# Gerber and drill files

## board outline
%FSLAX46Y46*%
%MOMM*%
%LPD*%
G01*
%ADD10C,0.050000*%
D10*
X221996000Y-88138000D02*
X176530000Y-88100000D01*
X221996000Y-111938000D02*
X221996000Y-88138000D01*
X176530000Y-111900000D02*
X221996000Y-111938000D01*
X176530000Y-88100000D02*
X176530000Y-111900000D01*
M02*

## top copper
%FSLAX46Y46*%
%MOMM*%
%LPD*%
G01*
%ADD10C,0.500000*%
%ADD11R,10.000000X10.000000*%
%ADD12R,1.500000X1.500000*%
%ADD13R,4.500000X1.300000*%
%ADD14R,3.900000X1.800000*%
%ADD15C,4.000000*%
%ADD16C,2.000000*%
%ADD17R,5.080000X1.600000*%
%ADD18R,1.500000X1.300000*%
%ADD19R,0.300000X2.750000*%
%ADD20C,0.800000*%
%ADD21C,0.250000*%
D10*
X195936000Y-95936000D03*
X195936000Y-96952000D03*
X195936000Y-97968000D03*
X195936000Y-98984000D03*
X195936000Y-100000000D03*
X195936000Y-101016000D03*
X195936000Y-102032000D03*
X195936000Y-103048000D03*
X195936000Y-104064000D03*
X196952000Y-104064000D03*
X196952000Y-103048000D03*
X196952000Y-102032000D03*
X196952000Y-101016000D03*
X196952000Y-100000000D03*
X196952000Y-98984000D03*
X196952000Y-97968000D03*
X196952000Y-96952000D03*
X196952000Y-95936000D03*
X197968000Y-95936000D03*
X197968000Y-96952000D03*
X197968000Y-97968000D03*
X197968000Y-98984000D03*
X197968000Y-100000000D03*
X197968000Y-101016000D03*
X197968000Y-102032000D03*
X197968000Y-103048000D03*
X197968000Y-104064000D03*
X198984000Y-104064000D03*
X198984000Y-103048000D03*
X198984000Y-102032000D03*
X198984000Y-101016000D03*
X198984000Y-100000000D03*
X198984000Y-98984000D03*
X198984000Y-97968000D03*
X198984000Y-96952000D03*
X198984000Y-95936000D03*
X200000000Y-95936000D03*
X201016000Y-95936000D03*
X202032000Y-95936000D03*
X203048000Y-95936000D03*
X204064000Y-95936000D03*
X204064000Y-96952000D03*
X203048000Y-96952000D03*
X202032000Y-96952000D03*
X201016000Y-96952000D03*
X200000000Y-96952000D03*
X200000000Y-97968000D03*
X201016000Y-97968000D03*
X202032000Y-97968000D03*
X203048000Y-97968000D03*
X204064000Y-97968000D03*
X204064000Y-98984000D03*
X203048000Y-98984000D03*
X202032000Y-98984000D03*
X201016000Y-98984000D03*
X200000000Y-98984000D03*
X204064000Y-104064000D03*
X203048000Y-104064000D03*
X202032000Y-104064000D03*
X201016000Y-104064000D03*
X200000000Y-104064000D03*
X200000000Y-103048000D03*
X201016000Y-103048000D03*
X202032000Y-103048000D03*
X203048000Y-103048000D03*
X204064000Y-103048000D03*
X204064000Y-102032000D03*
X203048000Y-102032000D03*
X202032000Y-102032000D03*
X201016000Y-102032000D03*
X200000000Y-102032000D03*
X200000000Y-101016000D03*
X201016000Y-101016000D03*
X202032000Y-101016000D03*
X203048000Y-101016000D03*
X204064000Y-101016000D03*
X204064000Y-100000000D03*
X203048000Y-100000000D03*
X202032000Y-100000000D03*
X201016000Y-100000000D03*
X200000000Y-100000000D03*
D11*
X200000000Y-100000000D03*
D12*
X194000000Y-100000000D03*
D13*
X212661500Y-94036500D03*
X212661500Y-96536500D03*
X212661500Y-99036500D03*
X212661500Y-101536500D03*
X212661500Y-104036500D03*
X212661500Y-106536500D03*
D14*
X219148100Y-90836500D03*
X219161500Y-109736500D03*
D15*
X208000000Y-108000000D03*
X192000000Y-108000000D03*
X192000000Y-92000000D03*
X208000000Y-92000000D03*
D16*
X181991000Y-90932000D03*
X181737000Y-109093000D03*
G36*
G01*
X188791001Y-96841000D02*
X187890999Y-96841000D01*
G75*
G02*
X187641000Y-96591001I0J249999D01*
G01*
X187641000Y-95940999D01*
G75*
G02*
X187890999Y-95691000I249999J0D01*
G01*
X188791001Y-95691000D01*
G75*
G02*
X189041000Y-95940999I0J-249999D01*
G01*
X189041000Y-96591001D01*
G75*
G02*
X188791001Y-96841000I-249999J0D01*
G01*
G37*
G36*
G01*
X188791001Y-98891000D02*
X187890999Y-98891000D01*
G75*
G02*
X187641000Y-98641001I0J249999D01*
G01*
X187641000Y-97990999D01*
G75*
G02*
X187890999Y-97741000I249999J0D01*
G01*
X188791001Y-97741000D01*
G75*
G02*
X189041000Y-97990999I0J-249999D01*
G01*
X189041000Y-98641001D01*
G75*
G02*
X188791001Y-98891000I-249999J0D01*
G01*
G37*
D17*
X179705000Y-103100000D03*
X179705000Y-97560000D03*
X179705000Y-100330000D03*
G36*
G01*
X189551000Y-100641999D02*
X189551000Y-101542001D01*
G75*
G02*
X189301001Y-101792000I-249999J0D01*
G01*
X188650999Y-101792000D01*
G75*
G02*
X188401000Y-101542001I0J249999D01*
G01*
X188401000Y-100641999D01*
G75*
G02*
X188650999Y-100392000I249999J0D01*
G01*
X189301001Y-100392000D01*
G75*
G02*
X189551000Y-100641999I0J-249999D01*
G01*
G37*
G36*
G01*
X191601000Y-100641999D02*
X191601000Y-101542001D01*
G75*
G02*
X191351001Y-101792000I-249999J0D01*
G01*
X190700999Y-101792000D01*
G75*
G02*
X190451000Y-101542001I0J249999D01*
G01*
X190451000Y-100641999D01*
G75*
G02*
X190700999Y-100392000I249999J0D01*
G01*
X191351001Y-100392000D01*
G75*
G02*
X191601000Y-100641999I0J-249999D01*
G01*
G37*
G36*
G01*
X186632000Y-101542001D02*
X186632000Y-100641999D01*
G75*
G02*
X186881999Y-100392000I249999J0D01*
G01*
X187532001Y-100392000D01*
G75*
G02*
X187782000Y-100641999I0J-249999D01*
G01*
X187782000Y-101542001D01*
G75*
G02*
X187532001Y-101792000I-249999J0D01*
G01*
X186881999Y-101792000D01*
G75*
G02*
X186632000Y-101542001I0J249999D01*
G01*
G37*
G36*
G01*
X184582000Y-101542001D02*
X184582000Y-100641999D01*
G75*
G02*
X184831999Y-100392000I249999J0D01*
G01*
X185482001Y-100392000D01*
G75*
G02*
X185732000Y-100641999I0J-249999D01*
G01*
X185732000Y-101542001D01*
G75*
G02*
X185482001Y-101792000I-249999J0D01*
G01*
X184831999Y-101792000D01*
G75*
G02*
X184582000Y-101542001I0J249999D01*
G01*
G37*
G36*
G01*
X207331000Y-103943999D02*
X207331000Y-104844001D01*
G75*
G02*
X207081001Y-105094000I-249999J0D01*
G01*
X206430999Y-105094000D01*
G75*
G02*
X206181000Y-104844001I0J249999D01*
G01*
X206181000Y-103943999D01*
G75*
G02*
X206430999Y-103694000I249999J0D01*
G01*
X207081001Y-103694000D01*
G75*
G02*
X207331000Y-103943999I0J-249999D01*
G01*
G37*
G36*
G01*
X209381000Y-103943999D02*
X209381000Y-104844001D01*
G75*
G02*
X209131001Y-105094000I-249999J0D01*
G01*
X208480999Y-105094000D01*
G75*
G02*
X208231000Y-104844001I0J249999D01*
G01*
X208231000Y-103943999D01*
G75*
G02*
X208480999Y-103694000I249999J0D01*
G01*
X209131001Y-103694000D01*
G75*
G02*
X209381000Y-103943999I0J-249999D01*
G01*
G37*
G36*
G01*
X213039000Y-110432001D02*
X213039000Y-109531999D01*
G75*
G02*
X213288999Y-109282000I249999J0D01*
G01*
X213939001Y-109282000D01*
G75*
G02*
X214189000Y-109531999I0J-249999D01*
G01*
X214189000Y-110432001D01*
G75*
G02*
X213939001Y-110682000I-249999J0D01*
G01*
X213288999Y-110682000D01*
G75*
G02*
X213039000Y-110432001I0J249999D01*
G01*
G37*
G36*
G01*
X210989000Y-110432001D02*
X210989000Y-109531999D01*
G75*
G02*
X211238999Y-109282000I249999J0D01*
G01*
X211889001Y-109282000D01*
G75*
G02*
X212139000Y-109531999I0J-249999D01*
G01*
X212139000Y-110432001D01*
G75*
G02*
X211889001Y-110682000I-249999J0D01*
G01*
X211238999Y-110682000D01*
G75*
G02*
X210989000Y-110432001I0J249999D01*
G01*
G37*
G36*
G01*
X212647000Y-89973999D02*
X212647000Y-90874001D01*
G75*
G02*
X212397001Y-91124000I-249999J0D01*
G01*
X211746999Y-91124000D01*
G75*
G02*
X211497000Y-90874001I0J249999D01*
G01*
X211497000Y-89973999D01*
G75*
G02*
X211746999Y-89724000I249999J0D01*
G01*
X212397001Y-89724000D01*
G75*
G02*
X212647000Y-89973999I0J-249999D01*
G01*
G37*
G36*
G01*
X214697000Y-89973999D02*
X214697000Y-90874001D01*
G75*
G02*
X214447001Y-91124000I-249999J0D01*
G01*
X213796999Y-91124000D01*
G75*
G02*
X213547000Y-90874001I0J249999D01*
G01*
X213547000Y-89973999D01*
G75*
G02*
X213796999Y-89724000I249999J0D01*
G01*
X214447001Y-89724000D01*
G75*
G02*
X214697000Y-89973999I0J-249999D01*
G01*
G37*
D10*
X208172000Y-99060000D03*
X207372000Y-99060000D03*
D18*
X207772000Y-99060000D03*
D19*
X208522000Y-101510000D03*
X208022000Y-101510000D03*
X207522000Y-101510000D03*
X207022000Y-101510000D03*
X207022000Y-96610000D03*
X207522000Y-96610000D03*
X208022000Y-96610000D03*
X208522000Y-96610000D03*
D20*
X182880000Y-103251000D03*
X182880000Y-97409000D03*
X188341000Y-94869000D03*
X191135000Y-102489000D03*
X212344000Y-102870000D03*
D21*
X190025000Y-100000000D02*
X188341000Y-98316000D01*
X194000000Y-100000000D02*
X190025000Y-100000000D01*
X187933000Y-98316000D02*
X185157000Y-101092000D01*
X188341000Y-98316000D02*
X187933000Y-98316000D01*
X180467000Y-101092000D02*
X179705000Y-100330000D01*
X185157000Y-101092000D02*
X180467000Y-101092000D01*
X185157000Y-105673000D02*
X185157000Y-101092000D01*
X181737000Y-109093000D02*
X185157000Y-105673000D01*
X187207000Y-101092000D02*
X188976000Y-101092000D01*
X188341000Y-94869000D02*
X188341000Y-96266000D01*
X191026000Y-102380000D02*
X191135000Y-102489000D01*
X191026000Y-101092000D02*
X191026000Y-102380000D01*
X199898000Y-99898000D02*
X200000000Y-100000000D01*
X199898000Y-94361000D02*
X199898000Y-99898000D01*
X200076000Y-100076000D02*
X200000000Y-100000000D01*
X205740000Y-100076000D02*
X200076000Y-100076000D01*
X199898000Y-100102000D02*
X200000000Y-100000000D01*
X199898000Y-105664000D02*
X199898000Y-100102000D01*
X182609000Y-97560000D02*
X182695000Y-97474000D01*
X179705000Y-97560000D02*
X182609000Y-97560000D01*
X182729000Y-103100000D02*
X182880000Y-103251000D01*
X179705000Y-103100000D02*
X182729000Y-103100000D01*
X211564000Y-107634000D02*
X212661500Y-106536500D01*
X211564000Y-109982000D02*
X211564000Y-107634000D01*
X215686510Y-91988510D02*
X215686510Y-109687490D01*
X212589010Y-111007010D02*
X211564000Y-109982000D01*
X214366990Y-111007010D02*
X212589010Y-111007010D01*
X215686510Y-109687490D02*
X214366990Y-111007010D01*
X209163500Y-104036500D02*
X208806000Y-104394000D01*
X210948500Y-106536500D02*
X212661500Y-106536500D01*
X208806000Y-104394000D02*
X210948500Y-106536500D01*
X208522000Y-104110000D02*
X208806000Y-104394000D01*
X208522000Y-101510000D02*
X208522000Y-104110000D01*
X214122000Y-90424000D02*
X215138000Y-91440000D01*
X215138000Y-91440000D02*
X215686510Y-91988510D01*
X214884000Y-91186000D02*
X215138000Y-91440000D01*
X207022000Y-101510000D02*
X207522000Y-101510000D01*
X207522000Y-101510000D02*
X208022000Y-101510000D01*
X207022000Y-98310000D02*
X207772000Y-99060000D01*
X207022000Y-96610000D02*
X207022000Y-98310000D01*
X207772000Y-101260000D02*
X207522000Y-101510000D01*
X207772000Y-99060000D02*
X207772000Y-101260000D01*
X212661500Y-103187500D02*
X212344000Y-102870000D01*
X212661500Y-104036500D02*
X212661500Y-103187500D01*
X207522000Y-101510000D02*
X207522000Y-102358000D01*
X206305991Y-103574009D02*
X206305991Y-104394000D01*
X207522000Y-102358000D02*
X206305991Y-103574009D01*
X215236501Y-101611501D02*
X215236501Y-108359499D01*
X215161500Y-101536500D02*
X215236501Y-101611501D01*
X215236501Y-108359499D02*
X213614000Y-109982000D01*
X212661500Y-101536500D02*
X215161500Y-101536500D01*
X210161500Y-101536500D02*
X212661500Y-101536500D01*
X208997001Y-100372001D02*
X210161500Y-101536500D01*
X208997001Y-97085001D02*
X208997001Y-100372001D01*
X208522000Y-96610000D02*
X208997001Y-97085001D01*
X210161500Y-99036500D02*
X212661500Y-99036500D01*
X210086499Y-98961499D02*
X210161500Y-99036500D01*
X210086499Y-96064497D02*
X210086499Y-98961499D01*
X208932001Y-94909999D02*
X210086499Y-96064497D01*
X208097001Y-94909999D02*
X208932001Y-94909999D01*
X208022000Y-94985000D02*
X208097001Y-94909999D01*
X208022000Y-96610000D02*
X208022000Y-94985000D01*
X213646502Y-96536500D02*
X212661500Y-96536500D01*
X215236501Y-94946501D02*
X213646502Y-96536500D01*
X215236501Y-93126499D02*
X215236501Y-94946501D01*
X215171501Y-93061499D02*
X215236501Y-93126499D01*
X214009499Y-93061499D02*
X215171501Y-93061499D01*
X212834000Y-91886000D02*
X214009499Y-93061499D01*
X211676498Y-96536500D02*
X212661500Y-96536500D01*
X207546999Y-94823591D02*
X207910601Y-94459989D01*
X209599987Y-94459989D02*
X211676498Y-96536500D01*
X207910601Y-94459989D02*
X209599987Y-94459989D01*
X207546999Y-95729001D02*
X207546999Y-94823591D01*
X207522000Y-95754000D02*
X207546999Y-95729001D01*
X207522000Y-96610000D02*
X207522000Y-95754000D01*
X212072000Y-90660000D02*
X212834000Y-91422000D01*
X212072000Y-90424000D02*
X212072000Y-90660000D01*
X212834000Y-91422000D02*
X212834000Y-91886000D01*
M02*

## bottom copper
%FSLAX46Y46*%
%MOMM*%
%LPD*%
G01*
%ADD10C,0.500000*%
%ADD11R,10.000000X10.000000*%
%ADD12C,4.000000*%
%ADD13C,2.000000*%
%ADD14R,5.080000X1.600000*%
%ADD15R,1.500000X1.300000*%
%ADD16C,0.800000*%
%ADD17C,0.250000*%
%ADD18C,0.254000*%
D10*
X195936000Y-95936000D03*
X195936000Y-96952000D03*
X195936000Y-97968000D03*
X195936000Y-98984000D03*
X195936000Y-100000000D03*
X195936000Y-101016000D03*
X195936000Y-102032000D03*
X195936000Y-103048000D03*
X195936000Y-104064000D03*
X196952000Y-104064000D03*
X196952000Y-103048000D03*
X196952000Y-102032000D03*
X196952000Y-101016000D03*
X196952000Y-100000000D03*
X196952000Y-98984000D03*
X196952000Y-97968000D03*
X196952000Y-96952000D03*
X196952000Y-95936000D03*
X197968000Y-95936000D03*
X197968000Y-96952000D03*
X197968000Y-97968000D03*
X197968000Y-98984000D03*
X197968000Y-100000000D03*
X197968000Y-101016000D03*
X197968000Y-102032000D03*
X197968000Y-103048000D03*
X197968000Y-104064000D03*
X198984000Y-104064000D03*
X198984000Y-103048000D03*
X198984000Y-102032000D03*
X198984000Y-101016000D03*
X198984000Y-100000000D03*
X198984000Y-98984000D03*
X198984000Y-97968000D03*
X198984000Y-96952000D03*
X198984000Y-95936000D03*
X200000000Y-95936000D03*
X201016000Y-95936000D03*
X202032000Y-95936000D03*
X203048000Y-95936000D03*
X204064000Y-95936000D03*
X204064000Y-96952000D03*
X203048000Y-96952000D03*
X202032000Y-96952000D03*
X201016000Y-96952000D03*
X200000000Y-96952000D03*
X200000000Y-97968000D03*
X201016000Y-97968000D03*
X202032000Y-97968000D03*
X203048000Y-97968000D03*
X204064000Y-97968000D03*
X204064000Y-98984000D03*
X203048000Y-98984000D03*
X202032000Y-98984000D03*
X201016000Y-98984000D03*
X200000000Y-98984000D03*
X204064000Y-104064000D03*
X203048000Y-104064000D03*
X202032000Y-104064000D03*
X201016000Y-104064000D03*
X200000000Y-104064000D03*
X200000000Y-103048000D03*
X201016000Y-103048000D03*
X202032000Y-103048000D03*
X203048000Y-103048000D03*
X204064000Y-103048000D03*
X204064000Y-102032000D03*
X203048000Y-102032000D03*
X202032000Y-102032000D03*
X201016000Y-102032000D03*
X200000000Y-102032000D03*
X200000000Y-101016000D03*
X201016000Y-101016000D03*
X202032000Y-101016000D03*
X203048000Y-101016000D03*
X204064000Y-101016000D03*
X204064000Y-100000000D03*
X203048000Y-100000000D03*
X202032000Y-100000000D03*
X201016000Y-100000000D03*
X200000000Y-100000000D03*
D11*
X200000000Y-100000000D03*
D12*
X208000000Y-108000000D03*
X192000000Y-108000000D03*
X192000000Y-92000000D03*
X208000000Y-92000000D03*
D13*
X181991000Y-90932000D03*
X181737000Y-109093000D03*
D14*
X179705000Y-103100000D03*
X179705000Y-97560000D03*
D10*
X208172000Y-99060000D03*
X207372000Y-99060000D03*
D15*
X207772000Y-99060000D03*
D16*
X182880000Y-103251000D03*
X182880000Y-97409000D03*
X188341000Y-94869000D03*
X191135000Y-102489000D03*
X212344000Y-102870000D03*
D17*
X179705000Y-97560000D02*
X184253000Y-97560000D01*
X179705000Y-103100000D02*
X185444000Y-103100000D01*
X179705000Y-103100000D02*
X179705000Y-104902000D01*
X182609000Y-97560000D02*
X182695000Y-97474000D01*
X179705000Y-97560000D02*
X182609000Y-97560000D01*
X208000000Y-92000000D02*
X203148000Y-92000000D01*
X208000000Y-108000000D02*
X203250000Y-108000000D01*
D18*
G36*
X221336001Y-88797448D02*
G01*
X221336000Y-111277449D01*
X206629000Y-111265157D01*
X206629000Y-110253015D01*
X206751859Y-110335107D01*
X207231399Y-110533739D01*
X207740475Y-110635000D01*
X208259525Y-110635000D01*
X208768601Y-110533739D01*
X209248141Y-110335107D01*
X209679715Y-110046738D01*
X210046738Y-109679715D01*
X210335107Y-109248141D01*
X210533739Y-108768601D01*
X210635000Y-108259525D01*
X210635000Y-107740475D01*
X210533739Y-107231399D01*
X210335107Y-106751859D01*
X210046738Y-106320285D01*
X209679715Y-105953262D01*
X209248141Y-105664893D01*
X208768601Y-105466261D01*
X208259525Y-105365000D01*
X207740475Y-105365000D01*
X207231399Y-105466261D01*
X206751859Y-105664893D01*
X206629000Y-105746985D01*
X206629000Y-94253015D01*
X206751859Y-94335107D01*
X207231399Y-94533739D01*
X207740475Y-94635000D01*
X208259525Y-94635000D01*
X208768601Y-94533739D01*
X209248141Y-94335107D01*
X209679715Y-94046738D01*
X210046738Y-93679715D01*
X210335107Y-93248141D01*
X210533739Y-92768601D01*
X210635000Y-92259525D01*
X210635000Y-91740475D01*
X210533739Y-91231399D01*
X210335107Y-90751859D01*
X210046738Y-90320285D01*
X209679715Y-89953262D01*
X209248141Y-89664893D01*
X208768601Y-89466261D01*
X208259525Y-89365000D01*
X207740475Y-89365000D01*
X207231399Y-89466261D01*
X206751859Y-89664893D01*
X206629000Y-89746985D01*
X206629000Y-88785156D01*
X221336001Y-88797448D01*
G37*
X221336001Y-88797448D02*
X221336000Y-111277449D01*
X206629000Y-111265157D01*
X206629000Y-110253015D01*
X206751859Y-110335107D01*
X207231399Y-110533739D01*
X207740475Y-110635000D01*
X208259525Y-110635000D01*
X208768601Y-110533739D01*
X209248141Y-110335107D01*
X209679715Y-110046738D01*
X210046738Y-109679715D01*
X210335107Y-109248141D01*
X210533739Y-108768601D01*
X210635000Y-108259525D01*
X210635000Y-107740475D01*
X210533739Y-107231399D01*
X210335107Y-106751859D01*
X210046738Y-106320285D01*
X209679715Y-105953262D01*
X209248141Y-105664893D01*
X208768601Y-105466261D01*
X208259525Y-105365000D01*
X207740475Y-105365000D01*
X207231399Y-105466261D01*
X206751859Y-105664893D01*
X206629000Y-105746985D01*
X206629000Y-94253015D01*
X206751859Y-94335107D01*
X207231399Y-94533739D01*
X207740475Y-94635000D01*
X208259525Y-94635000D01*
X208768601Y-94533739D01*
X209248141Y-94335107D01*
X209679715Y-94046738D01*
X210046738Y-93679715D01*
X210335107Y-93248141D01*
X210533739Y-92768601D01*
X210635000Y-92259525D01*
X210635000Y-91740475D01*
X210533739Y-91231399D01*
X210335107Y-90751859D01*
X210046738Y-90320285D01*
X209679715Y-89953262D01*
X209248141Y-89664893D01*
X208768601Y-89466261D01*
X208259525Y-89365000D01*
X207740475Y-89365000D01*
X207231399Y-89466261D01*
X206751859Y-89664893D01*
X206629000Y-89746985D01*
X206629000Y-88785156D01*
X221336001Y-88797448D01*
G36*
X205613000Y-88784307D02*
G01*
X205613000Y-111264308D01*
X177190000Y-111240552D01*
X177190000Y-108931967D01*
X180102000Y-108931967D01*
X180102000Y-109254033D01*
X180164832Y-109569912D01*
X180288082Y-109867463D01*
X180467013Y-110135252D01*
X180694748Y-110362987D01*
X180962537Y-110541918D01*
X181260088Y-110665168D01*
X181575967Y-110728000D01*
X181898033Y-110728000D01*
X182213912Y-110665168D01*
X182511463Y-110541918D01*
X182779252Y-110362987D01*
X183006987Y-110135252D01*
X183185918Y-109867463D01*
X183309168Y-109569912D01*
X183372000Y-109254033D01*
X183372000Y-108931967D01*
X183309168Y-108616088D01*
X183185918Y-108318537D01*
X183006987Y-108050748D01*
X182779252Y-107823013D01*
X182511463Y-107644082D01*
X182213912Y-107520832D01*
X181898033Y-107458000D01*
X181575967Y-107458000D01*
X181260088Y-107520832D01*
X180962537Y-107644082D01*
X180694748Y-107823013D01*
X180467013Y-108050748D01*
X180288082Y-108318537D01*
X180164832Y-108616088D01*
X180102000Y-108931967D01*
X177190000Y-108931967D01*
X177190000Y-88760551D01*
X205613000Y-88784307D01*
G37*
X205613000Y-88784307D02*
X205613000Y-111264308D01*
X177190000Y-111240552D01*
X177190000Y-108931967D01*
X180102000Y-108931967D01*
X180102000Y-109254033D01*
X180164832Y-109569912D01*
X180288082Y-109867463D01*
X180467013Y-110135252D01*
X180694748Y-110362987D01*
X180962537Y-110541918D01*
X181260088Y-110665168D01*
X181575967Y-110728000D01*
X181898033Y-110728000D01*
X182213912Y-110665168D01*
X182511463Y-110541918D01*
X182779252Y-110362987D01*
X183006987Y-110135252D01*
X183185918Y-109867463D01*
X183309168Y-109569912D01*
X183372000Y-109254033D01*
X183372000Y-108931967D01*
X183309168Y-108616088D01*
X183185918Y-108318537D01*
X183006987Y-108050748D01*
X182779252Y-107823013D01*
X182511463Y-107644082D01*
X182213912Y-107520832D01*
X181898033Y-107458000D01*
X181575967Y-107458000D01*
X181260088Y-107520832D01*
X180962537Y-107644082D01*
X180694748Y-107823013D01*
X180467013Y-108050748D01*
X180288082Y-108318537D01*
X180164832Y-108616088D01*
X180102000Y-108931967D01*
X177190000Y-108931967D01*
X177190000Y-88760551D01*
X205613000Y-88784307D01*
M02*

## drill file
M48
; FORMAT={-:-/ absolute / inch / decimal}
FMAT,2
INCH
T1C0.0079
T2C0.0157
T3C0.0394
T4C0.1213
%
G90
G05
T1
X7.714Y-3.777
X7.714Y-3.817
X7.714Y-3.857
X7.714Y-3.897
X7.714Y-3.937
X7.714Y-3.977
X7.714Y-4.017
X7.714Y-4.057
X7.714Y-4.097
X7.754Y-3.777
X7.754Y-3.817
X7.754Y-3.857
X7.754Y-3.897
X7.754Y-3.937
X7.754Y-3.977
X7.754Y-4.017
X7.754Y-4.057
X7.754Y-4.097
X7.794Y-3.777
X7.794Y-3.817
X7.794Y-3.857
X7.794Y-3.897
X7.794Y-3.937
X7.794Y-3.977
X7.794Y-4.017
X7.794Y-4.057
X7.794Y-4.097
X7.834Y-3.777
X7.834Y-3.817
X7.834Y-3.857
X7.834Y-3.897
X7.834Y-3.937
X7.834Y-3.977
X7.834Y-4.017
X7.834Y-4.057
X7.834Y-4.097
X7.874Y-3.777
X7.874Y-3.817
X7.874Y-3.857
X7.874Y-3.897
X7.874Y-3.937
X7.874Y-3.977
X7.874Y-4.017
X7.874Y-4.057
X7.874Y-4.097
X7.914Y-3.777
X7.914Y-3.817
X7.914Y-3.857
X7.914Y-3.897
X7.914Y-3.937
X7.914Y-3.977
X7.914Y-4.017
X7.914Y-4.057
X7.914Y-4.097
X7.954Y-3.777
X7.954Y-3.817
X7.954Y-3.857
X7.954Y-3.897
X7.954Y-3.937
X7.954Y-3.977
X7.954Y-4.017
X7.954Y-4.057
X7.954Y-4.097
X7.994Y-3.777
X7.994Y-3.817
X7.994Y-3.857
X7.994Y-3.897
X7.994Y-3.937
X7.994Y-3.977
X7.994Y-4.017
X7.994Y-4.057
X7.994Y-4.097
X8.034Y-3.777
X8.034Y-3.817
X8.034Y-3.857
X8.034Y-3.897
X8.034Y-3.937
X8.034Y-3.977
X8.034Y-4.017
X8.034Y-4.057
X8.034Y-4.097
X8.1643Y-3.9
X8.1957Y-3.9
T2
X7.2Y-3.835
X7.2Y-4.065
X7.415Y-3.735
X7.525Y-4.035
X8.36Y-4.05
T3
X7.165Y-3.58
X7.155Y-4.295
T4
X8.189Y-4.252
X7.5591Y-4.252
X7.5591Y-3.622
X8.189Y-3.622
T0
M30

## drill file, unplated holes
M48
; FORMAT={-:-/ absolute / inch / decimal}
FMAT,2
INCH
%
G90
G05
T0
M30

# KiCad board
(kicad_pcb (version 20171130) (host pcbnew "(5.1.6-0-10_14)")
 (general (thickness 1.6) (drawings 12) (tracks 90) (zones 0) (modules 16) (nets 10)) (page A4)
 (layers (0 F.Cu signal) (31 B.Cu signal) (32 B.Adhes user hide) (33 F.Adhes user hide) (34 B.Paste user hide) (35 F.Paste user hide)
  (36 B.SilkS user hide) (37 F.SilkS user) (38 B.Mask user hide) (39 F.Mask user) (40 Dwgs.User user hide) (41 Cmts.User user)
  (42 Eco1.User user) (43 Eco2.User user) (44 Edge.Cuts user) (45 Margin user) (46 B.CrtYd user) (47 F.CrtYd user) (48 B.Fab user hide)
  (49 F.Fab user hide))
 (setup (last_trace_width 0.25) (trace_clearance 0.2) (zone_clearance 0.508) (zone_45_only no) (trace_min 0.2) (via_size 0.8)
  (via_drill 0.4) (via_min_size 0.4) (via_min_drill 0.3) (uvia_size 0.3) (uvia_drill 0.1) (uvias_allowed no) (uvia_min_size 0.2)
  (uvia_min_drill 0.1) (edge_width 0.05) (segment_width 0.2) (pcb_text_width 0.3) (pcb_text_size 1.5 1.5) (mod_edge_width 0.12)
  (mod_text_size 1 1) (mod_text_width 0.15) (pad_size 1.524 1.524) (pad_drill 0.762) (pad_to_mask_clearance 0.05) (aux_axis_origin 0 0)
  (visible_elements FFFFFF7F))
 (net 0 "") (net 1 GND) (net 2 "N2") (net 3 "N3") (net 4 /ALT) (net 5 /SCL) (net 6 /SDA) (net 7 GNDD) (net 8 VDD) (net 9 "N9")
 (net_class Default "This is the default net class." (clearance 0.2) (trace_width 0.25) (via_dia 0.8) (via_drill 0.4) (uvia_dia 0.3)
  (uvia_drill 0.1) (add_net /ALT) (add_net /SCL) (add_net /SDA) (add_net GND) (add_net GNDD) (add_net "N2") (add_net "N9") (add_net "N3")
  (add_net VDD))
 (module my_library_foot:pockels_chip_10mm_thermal (layer F.Cu) (at 200 100)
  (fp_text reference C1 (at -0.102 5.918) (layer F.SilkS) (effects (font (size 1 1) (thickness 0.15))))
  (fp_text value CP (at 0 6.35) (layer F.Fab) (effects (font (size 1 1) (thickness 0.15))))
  (pad 2 thru_hole circle (at -4.064 -4.064) (size 0.5 0.5) (drill 0.2) (layers *.Cu *.Mask) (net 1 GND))
  (pad 2 thru_hole circle (at -4.064 -3.048) (size 0.5 0.5) (drill 0.2) (layers *.Cu *.Mask) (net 1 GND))
  (pad 2 thru_hole circle (at -4.064 -2.032) (size 0.5 0.5) (drill 0.2) (layers *.Cu *.Mask) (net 1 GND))
  (pad 2 thru_hole circle (at -4.064 -1.016) (size 0.5 0.5) (drill 0.2) (layers *.Cu *.Mask) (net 1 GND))
  (pad 2 thru_hole circle (at -4.064 0) (size 0.5 0.5) (drill 0.2) (layers *.Cu *.Mask) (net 1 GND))
  (pad 2 thru_hole circle (at -4.064 1.016) (size 0.5 0.5) (drill 0.2) (layers *.Cu *.Mask) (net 1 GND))
  (pad 2 thru_hole circle (at -4.064 2.032) (size 0.5 0.5) (drill 0.2) (layers *.Cu *.Mask) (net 1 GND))
  (pad 2 thru_hole circle (at -4.064 3.048) (size 0.5 0.5) (drill 0.2) (layers *.Cu *.Mask) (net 1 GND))
  (pad 2 thru_hole circle (at -4.064 4.064) (size 0.5 0.5) (drill 0.2) (layers *.Cu *.Mask) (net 1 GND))
  (pad 2 thru_hole circle (at -3.048 4.064) (size 0.5 0.5) (drill 0.2) (layers *.Cu *.Mask) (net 1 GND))
  (pad 2 thru_hole circle (at -3.048 3.048) (size 0.5 0.5) (drill 0.2) (layers *.Cu *.Mask) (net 1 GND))
  (pad 2 thru_hole circle (at -3.048 2.032) (size 0.5 0.5) (drill 0.2) (layers *.Cu *.Mask) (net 1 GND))
  (pad 2 thru_hole circle (at -3.048 1.016) (size 0.5 0.5) (drill 0.2) (layers *.Cu *.Mask) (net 1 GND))
  (pad 2 thru_hole circle (at -3.048 0) (size 0.5 0.5) (drill 0.2) (layers *.Cu *.Mask) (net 1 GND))
  (pad 2 thru_hole circle (at -3.048 -1.016) (size 0.5 0.5) (drill 0.2) (layers *.Cu *.Mask) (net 1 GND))
  (pad 2 thru_hole circle (at -3.048 -2.032) (size 0.5 0.5) (drill 0.2) (layers *.Cu *.Mask) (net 1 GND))
  (pad 2 thru_hole circle (at -3.048 -3.048) (size 0.5 0.5) (drill 0.2) (layers *.Cu *.Mask) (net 1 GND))
  (pad 2 thru_hole circle (at -3.048 -4.064) (size 0.5 0.5) (drill 0.2) (layers *.Cu *.Mask) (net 1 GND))
  (pad 2 thru_hole circle (at -2.032 -4.064) (size 0.5 0.5) (drill 0.2) (layers *.Cu *.Mask) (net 1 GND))
  (pad 2 thru_hole circle (at -2.032 -3.048) (size 0.5 0.5) (drill 0.2) (layers *.Cu *.Mask) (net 1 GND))
  (pad 2 thru_hole circle (at -2.032 -2.032) (size 0.5 0.5) (drill 0.2) (layers *.Cu *.Mask) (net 1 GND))
  (pad 2 thru_hole circle (at -2.032 -1.016) (size 0.5 0.5) (drill 0.2) (layers *.Cu *.Mask) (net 1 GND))
  (pad 2 thru_hole circle (at -2.032 0) (size 0.5 0.5) (drill 0.2) (layers *.Cu *.Mask) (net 1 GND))
  (pad 2 thru_hole circle (at -2.032 1.016) (size 0.5 0.5) (drill 0.2) (layers *.Cu *.Mask) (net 1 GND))
  (pad 2 thru_hole circle (at -2.032 2.032) (size 0.5 0.5) (drill 0.2) (layers *.Cu *.Mask) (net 1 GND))
  (pad 2 thru_hole circle (at -2.032 3.048) (size 0.5 0.5) (drill 0.2) (layers *.Cu *.Mask) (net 1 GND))
  (pad 2 thru_hole circle (at -2.032 4.064) (size 0.5 0.5) (drill 0.2) (layers *.Cu *.Mask) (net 1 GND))
  (pad 2 thru_hole circle (at -1.016 4.064) (size 0.5 0.5) (drill 0.2) (layers *.Cu *.Mask) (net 1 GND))
  (pad 2 thru_hole circle (at -1.016 3.048) (size 0.5 0.5) (drill 0.2) (layers *.Cu *.Mask) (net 1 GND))
  (pad 2 thru_hole circle (at -1.016 2.032) (size 0.5 0.5) (drill 0.2) (layers *.Cu *.Mask) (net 1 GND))
  (pad 2 thru_hole circle (at -1.016 1.016) (size 0.5 0.5) (drill 0.2) (layers *.Cu *.Mask) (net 1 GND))
  (pad 2 thru_hole circle (at -1.016 0) (size 0.5 0.5) (drill 0.2) (layers *.Cu *.Mask) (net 1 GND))
  (pad 2 thru_hole circle (at -1.016 -1.016) (size 0.5 0.5) (drill 0.2) (layers *.Cu *.Mask) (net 1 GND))
  (pad 2 thru_hole circle (at -1.016 -2.032) (size 0.5 0.5) (drill 0.2) (layers *.Cu *.Mask) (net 1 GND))
  (pad 2 thru_hole circle (at -1.016 -3.048) (size 0.5 0.5) (drill 0.2) (layers *.Cu *.Mask) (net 1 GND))
  (pad 2 thru_hole circle (at -1.016 -4.064) (size 0.5 0.5) (drill 0.2) (layers *.Cu *.Mask) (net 1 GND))
  (pad 2 thru_hole circle (at 0 -4.064) (size 0.5 0.5) (drill 0.2) (layers *.Cu *.Mask) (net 1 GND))
  (pad 2 thru_hole circle (at 1.016 -4.064) (size 0.5 0.5) (drill 0.2) (layers *.Cu *.Mask) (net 1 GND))
  (pad 2 thru_hole circle (at 2.032 -4.064) (size 0.5 0.5) (drill 0.2) (layers *.Cu *.Mask) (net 1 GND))
  (pad 2 thru_hole circle (at 3.048 -4.064) (size 0.5 0.5) (drill 0.2) (layers *.Cu *.Mask) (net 1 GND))
  (pad 2 thru_hole circle (at 4.064 -4.064) (size 0.5 0.5) (drill 0.2) (layers *.Cu *.Mask) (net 1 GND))
  (pad 2 thru_hole circle (at 4.064 -3.048) (size 0.5 0.5) (drill 0.2) (layers *.Cu *.Mask) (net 1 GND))
  (pad 2 thru_hole circle (at 3.048 -3.048) (size 0.5 0.5) (drill 0.2) (layers *.Cu *.Mask) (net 1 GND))
  (pad 2 thru_hole circle (at 2.032 -3.048) (size 0.5 0.5) (drill 0.2) (layers *.Cu *.Mask) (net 1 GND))
  (pad 2 thru_hole circle (at 1.016 -3.048) (size 0.5 0.5) (drill 0.2) (layers *.Cu *.Mask) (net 1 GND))
  (pad 2 thru_hole circle (at 0 -3.048) (size 0.5 0.5) (drill 0.2) (layers *.Cu *.Mask) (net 1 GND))
  (pad 2 thru_hole circle (at 0 -2.032) (size 0.5 0.5) (drill 0.2) (layers *.Cu *.Mask) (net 1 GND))
  (pad 2 thru_hole circle (at 1.016 -2.032) (size 0.5 0.5) (drill 0.2) (layers *.Cu *.Mask) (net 1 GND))
  (pad 2 thru_hole circle (at 2.032 -2.032) (size 0.5 0.5) (drill 0.2) (layers *.Cu *.Mask) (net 1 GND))
  (pad 2 thru_hole circle (at 3.048 -2.032) (size 0.5 0.5) (drill 0.2) (layers *.Cu *.Mask) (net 1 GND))
  (pad 2 thru_hole circle (at 4.064 -2.032) (size 0.5 0.5) (drill 0.2) (layers *.Cu *.Mask) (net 1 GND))
  (pad 2 thru_hole circle (at 4.064 -1.016) (size 0.5 0.5) (drill 0.2) (layers *.Cu *.Mask) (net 1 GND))
  (pad 2 thru_hole circle (at 3.048 -1.016) (size 0.5 0.5) (drill 0.2) (layers *.Cu *.Mask) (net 1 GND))
  (pad 2 thru_hole circle (at 2.032 -1.016) (size 0.5 0.5) (drill 0.2) (layers *.Cu *.Mask) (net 1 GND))
  (pad 2 thru_hole circle (at 1.016 -1.016) (size 0.5 0.5) (drill 0.2) (layers *.Cu *.Mask) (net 1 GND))
  (pad 2 thru_hole circle (at 0 -1.016) (size 0.5 0.5) (drill 0.2) (layers *.Cu *.Mask) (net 1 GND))
  (pad 2 thru_hole circle (at 4.064 4.064) (size 0.5 0.5) (drill 0.2) (layers *.Cu *.Mask) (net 1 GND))
  (pad 2 thru_hole circle (at 3.048 4.064) (size 0.5 0.5) (drill 0.2) (layers *.Cu *.Mask) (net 1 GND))
  (pad 2 thru_hole circle (at 2.032 4.064) (size 0.5 0.5) (drill 0.2) (layers *.Cu *.Mask) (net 1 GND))
  (pad 2 thru_hole circle (at 1.016 4.064) (size 0.5 0.5) (drill 0.2) (layers *.Cu *.Mask) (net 1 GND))
  (pad 2 thru_hole circle (at 0 4.064) (size 0.5 0.5) (drill 0.2) (layers *.Cu *.Mask) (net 1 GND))
  (pad 2 thru_hole circle (at 0 3.048) (size 0.5 0.5) (drill 0.2) (layers *.Cu *.Mask) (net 1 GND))
  (pad 2 thru_hole circle (at 1.016 3.048) (size 0.5 0.5) (drill 0.2) (layers *.Cu *.Mask) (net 1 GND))
  (pad 2 thru_hole circle (at 2.032 3.048) (size 0.5 0.5) (drill 0.2) (layers *.Cu *.Mask) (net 1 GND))
  (pad 2 thru_hole circle (at 3.048 3.048) (size 0.5 0.5) (drill 0.2) (layers *.Cu *.Mask) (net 1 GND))
  (pad 2 thru_hole circle (at 4.064 3.048) (size 0.5 0.5) (drill 0.2) (layers *.Cu *.Mask) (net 1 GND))
  (pad 2 thru_hole circle (at 4.064 2.032) (size 0.5 0.5) (drill 0.2) (layers *.Cu *.Mask) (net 1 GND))
  (pad 2 thru_hole circle (at 3.048 2.032) (size 0.5 0.5) (drill 0.2) (layers *.Cu *.Mask) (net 1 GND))
  (pad 2 thru_hole circle (at 2.032 2.032) (size 0.5 0.5) (drill 0.2) (layers *.Cu *.Mask) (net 1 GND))
  (pad 2 thru_hole circle (at 1.016 2.032) (size 0.5 0.5) (drill 0.2) (layers *.Cu *.Mask) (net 1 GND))
  (pad 2 thru_hole circle (at 0 2.032) (size 0.5 0.5) (drill 0.2) (layers *.Cu *.Mask) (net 1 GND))
  (pad 2 thru_hole circle (at 0 1.016) (size 0.5 0.5) (drill 0.2) (layers *.Cu *.Mask) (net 1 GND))
  (pad 2 thru_hole circle (at 1.016 1.016) (size 0.5 0.5) (drill 0.2) (layers *.Cu *.Mask) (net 1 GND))
  (pad 2 thru_hole circle (at 2.032 1.016) (size 0.5 0.5) (drill 0.2) (layers *.Cu *.Mask) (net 1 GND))
  (pad 2 thru_hole circle (at 3.048 1.016) (size 0.5 0.5) (drill 0.2) (layers *.Cu *.Mask) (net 1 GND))
  (pad 2 thru_hole circle (at 4.064 1.016) (size 0.5 0.5) (drill 0.2) (layers *.Cu *.Mask) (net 1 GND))
  (pad 2 thru_hole circle (at 4.064 0) (size 0.5 0.5) (drill 0.2) (layers *.Cu *.Mask) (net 1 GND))
  (pad 2 thru_hole circle (at 3.048 0) (size 0.5 0.5) (drill 0.2) (layers *.Cu *.Mask) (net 1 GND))
  (pad 2 thru_hole circle (at 2.032 0) (size 0.5 0.5) (drill 0.2) (layers *.Cu *.Mask) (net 1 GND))
  (pad 2 thru_hole circle (at 1.016 0) (size 0.5 0.5) (drill 0.2) (layers *.Cu *.Mask) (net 1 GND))
  (pad 2 thru_hole circle (at 0 0) (size 0.5 0.5) (drill 0.2) (layers *.Cu *.Mask) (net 1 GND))
  (pad 2 smd rect (at 0 0) (size 10 10) (layers B.Cu B.Paste B.Mask) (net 1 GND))
  (pad 2 smd rect (at 0 0) (size 10 10) (layers F.Cu F.Paste F.Mask) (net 1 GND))
  (pad 1 smd rect (at -6 0) (size 1.5 1.5) (layers F.Cu F.Paste F.Mask) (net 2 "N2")))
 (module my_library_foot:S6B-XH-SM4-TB (layer F.Cu) (at 219.1615 109.7365 90)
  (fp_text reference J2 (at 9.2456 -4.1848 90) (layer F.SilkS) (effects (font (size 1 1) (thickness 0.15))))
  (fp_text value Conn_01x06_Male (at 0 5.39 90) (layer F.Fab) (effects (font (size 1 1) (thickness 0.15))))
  (pad 6 smd rect (at 15.7 -6.5 90) (size 1.3 4.5) (layers F.Cu F.Paste F.Mask) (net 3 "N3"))
  (pad 5 smd rect (at 13.2 -6.5 90) (size 1.3 4.5) (layers F.Cu F.Paste F.Mask) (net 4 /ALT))
  (pad 4 smd rect (at 10.7 -6.5 90) (size 1.3 4.5) (layers F.Cu F.Paste F.Mask) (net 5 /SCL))
  (pad 3 smd rect (at 8.2 -6.5 90) (size 1.3 4.5) (layers F.Cu F.Paste F.Mask) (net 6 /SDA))
  (pad 2 smd rect (at 5.7 -6.5 90) (size 1.3 4.5) (layers F.Cu F.Paste F.Mask) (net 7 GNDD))
  (pad 1 smd rect (at 3.2 -6.5 90) (size 1.3 4.5) (layers F.Cu F.Paste F.Mask) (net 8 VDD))
  (pad MP smd rect (at 18.9 -0.0134 90) (size 1.8 3.9) (layers F.Cu F.Paste F.Mask))
  (pad MP smd rect (at 0 0 90) (size 1.8 3.9) (layers F.Cu F.Paste F.Mask)))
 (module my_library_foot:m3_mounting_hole (layer F.Cu) (at 208 108)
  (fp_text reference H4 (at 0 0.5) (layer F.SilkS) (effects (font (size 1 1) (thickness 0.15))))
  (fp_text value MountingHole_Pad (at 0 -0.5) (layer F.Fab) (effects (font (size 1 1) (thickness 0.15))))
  (pad 1 thru_hole circle (at 0 0) (size 4 4) (drill 3.08) (layers *.Cu *.Mask) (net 1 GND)))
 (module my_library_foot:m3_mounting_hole (layer F.Cu) (at 192 108)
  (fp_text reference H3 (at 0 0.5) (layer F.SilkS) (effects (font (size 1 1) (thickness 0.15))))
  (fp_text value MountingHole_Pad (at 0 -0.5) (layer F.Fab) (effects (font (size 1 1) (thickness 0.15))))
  (pad 1 thru_hole circle (at 0 0) (size 4 4) (drill 3.08) (layers *.Cu *.Mask) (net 1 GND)))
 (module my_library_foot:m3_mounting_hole (layer F.Cu) (at 192 92)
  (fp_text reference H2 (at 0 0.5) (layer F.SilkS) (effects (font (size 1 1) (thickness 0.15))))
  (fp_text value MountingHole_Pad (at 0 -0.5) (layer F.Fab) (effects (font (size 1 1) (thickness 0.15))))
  (pad 1 thru_hole circle (at 0 0) (size 4 4) (drill 3.08) (layers *.Cu *.Mask) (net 1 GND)))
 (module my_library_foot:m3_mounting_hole (layer F.Cu) (at 208 92)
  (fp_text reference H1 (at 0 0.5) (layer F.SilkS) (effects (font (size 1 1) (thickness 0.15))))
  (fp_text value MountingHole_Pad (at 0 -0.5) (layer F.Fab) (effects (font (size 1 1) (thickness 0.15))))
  (pad 1 thru_hole circle (at 0 0) (size 4 4) (drill 3.08) (layers *.Cu *.Mask) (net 1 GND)))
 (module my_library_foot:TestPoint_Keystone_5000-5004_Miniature (layer F.Cu) (at 181.991 90.932)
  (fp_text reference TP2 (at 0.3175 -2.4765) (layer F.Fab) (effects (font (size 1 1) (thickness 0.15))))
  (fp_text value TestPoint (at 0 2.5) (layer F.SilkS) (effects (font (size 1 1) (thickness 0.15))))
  (pad 1 thru_hole circle (at 0 0) (size 2 2) (drill 1) (layers *.Cu *.Mask) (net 1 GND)))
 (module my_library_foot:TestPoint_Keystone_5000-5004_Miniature (layer F.Cu) (at 181.737 109.093)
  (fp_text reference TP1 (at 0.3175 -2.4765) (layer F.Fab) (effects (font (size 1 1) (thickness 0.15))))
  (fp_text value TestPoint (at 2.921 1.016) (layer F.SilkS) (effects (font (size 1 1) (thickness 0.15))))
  (pad 1 thru_hole circle (at 0 0) (size 2 2) (drill 1) (layers *.Cu *.Mask) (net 2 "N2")))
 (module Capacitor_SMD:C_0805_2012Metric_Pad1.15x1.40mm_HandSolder (layer F.Cu) (at 188.341 97.291 90)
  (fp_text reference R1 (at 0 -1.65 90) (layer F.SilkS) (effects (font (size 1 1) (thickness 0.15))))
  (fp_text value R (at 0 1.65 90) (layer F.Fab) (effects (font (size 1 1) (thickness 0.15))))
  (pad 2 smd roundrect (at 1.025 0 90) (size 1.15 1.4) (layers F.Cu F.Paste F.Mask) (roundrect_rratio 0.217391) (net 1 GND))
  (pad 1 smd roundrect (at -1.025 0 90) (size 1.15 1.4) (layers F.Cu F.Paste F.Mask) (roundrect_rratio 0.217391) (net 2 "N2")))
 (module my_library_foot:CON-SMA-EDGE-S (layer F.Cu) (at 181.425 100.33)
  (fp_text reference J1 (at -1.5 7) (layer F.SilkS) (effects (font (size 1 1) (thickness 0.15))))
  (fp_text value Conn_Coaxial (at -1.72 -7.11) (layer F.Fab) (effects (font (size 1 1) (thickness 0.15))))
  (pad 2 smd rect (at -1.72 2.77) (size 5.08 1.6) (layers B.Cu B.Paste B.Mask) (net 1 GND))
  (pad 2 smd rect (at -1.72 -2.77) (size 5.08 1.6) (layers B.Cu B.Paste B.Mask) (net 1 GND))
  (pad 2 smd rect (at -1.72 2.77) (size 5.08 1.6) (layers F.Cu F.Paste F.Mask) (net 1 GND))
  (pad 2 smd rect (at -1.72 -2.77) (size 5.08 1.6) (layers F.Cu F.Paste F.Mask) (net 1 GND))
  (pad 1 smd rect (at -1.72 0) (size 5.08 1.6) (layers F.Cu F.Paste F.Mask) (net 2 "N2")))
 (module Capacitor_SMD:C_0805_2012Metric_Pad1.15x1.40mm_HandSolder (layer F.Cu) (at 190.001 101.092 180)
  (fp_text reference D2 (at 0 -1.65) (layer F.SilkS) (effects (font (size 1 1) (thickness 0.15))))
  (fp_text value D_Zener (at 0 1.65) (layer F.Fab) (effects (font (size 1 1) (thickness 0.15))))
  (pad 2 smd roundrect (at 1.025 0 180) (size 1.15 1.4) (layers F.Cu F.Paste F.Mask) (roundrect_rratio 0.217391) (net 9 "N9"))
  (pad 1 smd roundrect (at -1.025 0 180) (size 1.15 1.4) (layers F.Cu F.Paste F.Mask) (roundrect_rratio 0.217391) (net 1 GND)))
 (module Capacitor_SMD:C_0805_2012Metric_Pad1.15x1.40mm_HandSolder (layer F.Cu) (at 186.182 101.092)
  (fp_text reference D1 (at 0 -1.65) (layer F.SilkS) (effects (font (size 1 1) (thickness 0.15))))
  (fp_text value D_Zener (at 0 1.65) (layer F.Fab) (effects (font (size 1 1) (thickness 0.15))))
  (pad 2 smd roundrect (at 1.025 0) (size 1.15 1.4) (layers F.Cu F.Paste F.Mask) (roundrect_rratio 0.217391) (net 9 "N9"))
  (pad 1 smd roundrect (at -1.025 0) (size 1.15 1.4) (layers F.Cu F.Paste F.Mask) (roundrect_rratio 0.217391) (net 2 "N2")))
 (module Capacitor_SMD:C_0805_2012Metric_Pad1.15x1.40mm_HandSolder (layer F.Cu) (at 207.781 104.394 180)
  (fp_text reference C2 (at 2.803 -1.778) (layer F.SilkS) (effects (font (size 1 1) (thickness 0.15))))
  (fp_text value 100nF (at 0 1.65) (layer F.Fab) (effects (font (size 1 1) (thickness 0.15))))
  (pad 2 smd roundrect (at 1.025 0 180) (size 1.15 1.4) (layers F.Cu F.Paste F.Mask) (roundrect_rratio 0.217391) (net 7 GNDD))
  (pad 1 smd roundrect (at -1.025 0 180) (size 1.15 1.4) (layers F.Cu F.Paste F.Mask) (roundrect_rratio 0.217391) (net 8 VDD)))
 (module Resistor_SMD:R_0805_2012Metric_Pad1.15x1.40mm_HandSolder (layer F.Cu) (at 212.589 109.982)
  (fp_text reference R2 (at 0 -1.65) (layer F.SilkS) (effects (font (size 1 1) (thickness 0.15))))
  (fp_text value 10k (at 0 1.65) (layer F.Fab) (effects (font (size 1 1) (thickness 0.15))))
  (pad 2 smd roundrect (at 1.025 0) (size 1.15 1.4) (layers F.Cu F.Paste F.Mask) (roundrect_rratio 0.217391) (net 6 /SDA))
  (pad 1 smd roundrect (at -1.025 0) (size 1.15 1.4) (layers F.Cu F.Paste F.Mask) (roundrect_rratio 0.217391) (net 8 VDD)))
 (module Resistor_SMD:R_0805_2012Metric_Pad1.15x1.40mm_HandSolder (layer F.Cu) (at 213.097 90.424 180)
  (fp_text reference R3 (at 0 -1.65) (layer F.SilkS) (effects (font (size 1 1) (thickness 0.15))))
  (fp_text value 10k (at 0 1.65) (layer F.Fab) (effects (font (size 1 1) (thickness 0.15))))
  (pad 2 smd roundrect (at 1.025 0 180) (size 1.15 1.4) (layers F.Cu F.Paste F.Mask) (roundrect_rratio 0.217391) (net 4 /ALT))
  (pad 1 smd roundrect (at -1.025 0 180) (size 1.15 1.4) (layers F.Cu F.Paste F.Mask) (roundrect_rratio 0.217391) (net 8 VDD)))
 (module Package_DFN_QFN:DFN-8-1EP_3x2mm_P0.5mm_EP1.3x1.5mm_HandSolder (layer F.Cu) (at 207.772 99.06 270)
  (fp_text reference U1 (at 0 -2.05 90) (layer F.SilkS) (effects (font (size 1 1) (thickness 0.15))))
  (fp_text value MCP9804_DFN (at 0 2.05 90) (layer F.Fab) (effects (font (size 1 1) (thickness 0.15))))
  (pad 9 thru_hole circle (at 0 -0.4 270) (size 0.5 0.5) (drill 0.2) (layers *.Cu *.Mask) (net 7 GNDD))
  (pad 9 thru_hole circle (at 0 0.4 270) (size 0.5 0.5) (drill 0.2) (layers *.Cu *.Mask) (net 7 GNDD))
  (pad 9 smd rect (at 0 0 270) (size 1.3 1.5) (layers B.Cu B.Paste B.Mask) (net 7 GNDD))
  (pad "" smd rect (at 0.325 0.375 270) (size 0.5 0.6) (layers F.Paste))
  (pad "" smd rect (at 0.325 -0.375 270) (size 0.5 0.6) (layers F.Paste))
  (pad "" smd rect (at -0.325 0.375 270) (size 0.5 0.6) (layers F.Paste))
  (pad "" smd rect (at -0.325 -0.375 270) (size 0.5 0.6) (layers F.Paste))
  (pad 9 smd rect (at 0 0 270) (size 1.3 1.5) (layers F.Cu F.Mask) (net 7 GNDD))
  (pad 8 smd rect (at 2.45 -0.75 270) (size 2.75 0.3) (layers F.Cu F.Paste F.Mask) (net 8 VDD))
  (pad 7 smd rect (at 2.45 -0.25 270) (size 2.75 0.3) (layers F.Cu F.Paste F.Mask) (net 7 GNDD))
  (pad 6 smd rect (at 2.45 0.25 270) (size 2.75 0.3) (layers F.Cu F.Paste F.Mask) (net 7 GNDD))
  (pad 5 smd rect (at 2.45 0.75 270) (size 2.75 0.3) (layers F.Cu F.Paste F.Mask) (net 7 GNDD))
  (pad 4 smd rect (at -2.45 0.75 270) (size 2.75 0.3) (layers F.Cu F.Paste F.Mask) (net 7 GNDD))
  (pad 3 smd rect (at -2.45 0.25 270) (size 2.75 0.3) (layers F.Cu F.Paste F.Mask) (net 4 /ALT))
  (pad 2 smd rect (at -2.45 -0.25 270) (size 2.75 0.3) (layers F.Cu F.Paste F.Mask) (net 5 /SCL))
  (pad 1 smd rect (at -2.45 -0.75 270) (size 2.75 0.3) (layers F.Cu F.Paste F.Mask) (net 6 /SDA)))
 (gr_line (start 221.996 88.138) (end 176.53 88.1) (layer Edge.Cuts) (width 0.05))
 (gr_line (start 221.996 111.938) (end 221.996 88.138) (layer Edge.Cuts) (width 0.05))
 (gr_line (start 176.53 111.9) (end 221.996 111.938) (layer Edge.Cuts) (width 0.05))
 (gr_line (start 176.53 88.1) (end 176.53 111.9) (layer Edge.Cuts) (width 0.05))
 (segment (start 190.025 100) (end 188.341 98.316) (width 0.25) (layer F.Cu) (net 2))
 (segment (start 194 100) (end 190.025 100) (width 0.25) (layer F.Cu) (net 2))
 (segment (start 187.933 98.316) (end 185.157 101.092) (width 0.25) (layer F.Cu) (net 2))
 (segment (start 188.341 98.316) (end 187.933 98.316) (width 0.25) (layer F.Cu) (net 2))
 (segment (start 180.467 101.092) (end 179.705 100.33) (width 0.25) (layer F.Cu) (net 2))
 (segment (start 185.157 101.092) (end 180.467 101.092) (width 0.25) (layer F.Cu) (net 2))
 (segment (start 185.157 105.673) (end 185.157 101.092) (width 0.25) (layer F.Cu) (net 2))
 (segment (start 181.737 109.093) (end 185.157 105.673) (width 0.25) (layer F.Cu) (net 2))
 (segment (start 187.207 101.092) (end 188.976 101.092) (width 0.25) (layer F.Cu) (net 9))
 (via (at 182.88 103.251) (size 0.8) (drill 0.4) (layers F.Cu B.Cu) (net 1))
 (via (at 182.88 97.409) (size 0.8) (drill 0.4) (layers F.Cu B.Cu) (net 1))
 (via (at 188.341 94.869) (size 0.8) (drill 0.4) (layers F.Cu B.Cu) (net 1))
 (via (at 191.135 102.489) (size 0.8) (drill 0.4) (layers F.Cu B.Cu) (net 1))
 (segment (start 188.341 94.869) (end 188.341 96.266) (width 0.25) (layer F.Cu) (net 1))
 (segment (start 191.026 102.38) (end 191.135 102.489) (width 0.25) (layer F.Cu) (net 1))
 (segment (start 191.026 101.092) (end 191.026 102.38) (width 0.25) (layer F.Cu) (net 1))
 (segment (start 199.898 99.898) (end 200 100) (width 0.25) (layer F.Cu) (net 1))
 (segment (start 199.898 94.361) (end 199.898 99.898) (width 0.25) (layer F.Cu) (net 1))
 (segment (start 200.076 100.076) (end 200 100) (width 0.25) (layer F.Cu) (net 1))
 (segment (start 205.74 100.076) (end 200.076 100.076) (width 0.25) (layer F.Cu) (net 1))
 (segment (start 199.898 100.102) (end 200 100) (width 0.25) (layer F.Cu) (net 1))
 (segment (start 199.898 105.664) (end 199.898 100.102) (width 0.25) (layer F.Cu) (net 1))
 (segment (start 179.705 97.56) (end 184.253 97.56) (width 0.25) (layer B.Cu) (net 1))
 (segment (start 179.705 103.1) (end 185.444 103.1) (width 0.25) (layer B.Cu) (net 1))
 (segment (start 179.705 103.1) (end 179.705 104.902) (width 0.25) (layer B.Cu) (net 1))
 (segment (start 182.609 97.56) (end 182.695 97.474) (width 0.25) (layer B.Cu) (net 1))
 (segment (start 179.705 97.56) (end 182.609 97.56) (width 0.25) (layer B.Cu) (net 1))
 (segment (start 182.609 97.56) (end 182.695 97.474) (width 0.25) (layer F.Cu) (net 1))
 (segment (start 179.705 97.56) (end 182.609 97.56) (width 0.25) (layer F.Cu) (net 1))
 (segment (start 182.729 103.1) (end 182.88 103.251) (width 0.25) (layer F.Cu) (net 1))
 (segment (start 179.705 103.1) (end 182.729 103.1) (width 0.25) (layer F.Cu) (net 1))
 (segment (start 208 92) (end 203.148 92) (width 0.25) (layer B.Cu) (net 1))
 (segment (start 208 108) (end 203.25 108) (width 0.25) (layer B.Cu) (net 1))
 (segment (start 211.564 107.634) (end 212.6615 106.5365) (width 0.25) (layer F.Cu) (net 8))
 (segment (start 211.564 109.982) (end 211.564 107.634) (width 0.25) (layer F.Cu) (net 8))
 (segment (start 215.68651 91.98851) (end 215.68651 109.68749) (width 0.25) (layer F.Cu) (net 8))
 (segment (start 212.58901 111.00701) (end 211.564 109.982) (width 0.25) (layer F.Cu) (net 8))
 (segment (start 214.36699 111.00701) (end 212.58901 111.00701) (width 0.25) (layer F.Cu) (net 8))
 (segment (start 215.68651 109.68749) (end 214.36699 111.00701) (width 0.25) (layer F.Cu) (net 8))
 (segment (start 209.1635 104.0365) (end 208.806 104.394) (width 0.25) (layer F.Cu) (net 8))
 (segment (start 210.9485 106.5365) (end 212.6615 106.5365) (width 0.25) (layer F.Cu) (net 8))
 (segment (start 208.806 104.394) (end 210.9485 106.5365) (width 0.25) (layer F.Cu) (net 8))
 (segment (start 208.522 104.11) (end 208.806 104.394) (width 0.25) (layer F.Cu) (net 8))
 (segment (start 208.522 101.51) (end 208.522 104.11) (width 0.25) (layer F.Cu) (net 8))
 (segment (start 214.122 90.424) (end 215.138 91.44) (width 0.25) (layer F.Cu) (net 8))
 (segment (start 215.138 91.44) (end 215.68651 91.98851) (width 0.25) (layer F.Cu) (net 8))
 (segment (start 214.884 91.186) (end 215.138 91.44) (width 0.25) (layer F.Cu) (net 8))
 (segment (start 207.022 101.51) (end 207.522 101.51) (width 0.25) (layer F.Cu) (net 7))
 (segment (start 207.522 101.51) (end 208.022 101.51) (width 0.25) (layer F.Cu) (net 7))
 (segment (start 207.022 98.31) (end 207.772 99.06) (width 0.25) (layer F.Cu) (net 7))
 (segment (start 207.022 96.61) (end 207.022 98.31) (width 0.25) (layer F.Cu) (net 7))
 (segment (start 207.772 101.26) (end 207.522 101.51) (width 0.25) (layer F.Cu) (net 7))
 (segment (start 207.772 99.06) (end 207.772 101.26) (width 0.25) (layer F.Cu) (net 7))
 (segment (start 212.6615 103.1875) (end 212.344 102.87) (width 0.25) (layer F.Cu) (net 7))
 (via (at 212.344 102.87) (size 0.8) (drill 0.4) (layers F.Cu B.Cu) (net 7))
 (segment (start 212.6615 104.0365) (end 212.6615 103.1875) (width 0.25) (layer F.Cu) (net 7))
 (segment (start 207.522 101.51) (end 207.522 102.358) (width 0.25) (layer F.Cu) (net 7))
 (segment (start 206.305991 103.574009) (end 206.305991 104.394) (width 0.25) (layer F.Cu) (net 7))
 (segment (start 207.522 102.358) (end 206.305991 103.574009) (width 0.25) (layer F.Cu) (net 7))
 (segment (start 215.236501 101.611501) (end 215.236501 108.359499) (width 0.25) (layer F.Cu) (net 6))
 (segment (start 215.1615 101.5365) (end 215.236501 101.611501) (width 0.25) (layer F.Cu) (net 6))
 (segment (start 215.236501 108.359499) (end 213.614 109.982) (width 0.25) (layer F.Cu) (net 6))
 (segment (start 212.6615 101.5365) (end 215.1615 101.5365) (width 0.25) (layer F.Cu) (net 6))
 (segment (start 210.1615 101.5365) (end 212.6615 101.5365) (width 0.25) (layer F.Cu) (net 6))
 (segment (start 208.997001 100.372001) (end 210.1615 101.5365) (width 0.25) (layer F.Cu) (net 6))
 (segment (start 208.997001 97.085001) (end 208.997001 100.372001) (width 0.25) (layer F.Cu) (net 6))
 (segment (start 208.522 96.61) (end 208.997001 97.085001) (width 0.25) (layer F.Cu) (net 6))
 (segment (start 210.1615 99.0365) (end 212.6615 99.0365) (width 0.25) (layer F.Cu) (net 5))
 (segment (start 210.086499 98.961499) (end 210.1615 99.0365) (width 0.25) (layer F.Cu) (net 5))
 (segment (start 210.086499 96.064497) (end 210.086499 98.961499) (width 0.25) (layer F.Cu) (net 5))
 (segment (start 208.932001 94.909999) (end 210.086499 96.064497) (width 0.25) (layer F.Cu) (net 5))
 (segment (start 208.097001 94.909999) (end 208.932001 94.909999) (width 0.25) (layer F.Cu) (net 5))
 (segment (start 208.022 94.985) (end 208.097001 94.909999) (width 0.25) (layer F.Cu) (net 5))
 (segment (start 208.022 96.61) (end 208.022 94.985) (width 0.25) (layer F.Cu) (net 5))
 (segment (start 213.646502 96.5365) (end 212.6615 96.5365) (width 0.25) (layer F.Cu) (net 4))
 (segment (start 215.236501 94.946501) (end 213.646502 96.5365) (width 0.25) (layer F.Cu) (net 4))
 (segment (start 215.236501 93.126499) (end 215.236501 94.946501) (width 0.25) (layer F.Cu) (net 4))
 (segment (start 215.171501 93.061499) (end 215.236501 93.126499) (width 0.25) (layer F.Cu) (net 4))
 (segment (start 214.009499 93.061499) (end 215.171501 93.061499) (width 0.25) (layer F.Cu) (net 4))
 (segment (start 212.834 91.886) (end 214.009499 93.061499) (width 0.25) (layer F.Cu) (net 4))
 (segment (start 211.676498 96.5365) (end 212.6615 96.5365) (width 0.25) (layer F.Cu) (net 4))
 (segment (start 207.546999 94.823591) (end 207.910601 94.459989) (width 0.25) (layer F.Cu) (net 4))
 (segment (start 209.599987 94.459989) (end 211.676498 96.5365) (width 0.25) (layer F.Cu) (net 4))
 (segment (start 207.910601 94.459989) (end 209.599987 94.459989) (width 0.25) (layer F.Cu) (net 4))
 (segment (start 207.546999 95.729001) (end 207.546999 94.823591) (width 0.25) (layer F.Cu) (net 4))
 (segment (start 207.522 95.754) (end 207.546999 95.729001) (width 0.25) (layer F.Cu) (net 4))
 (segment (start 207.522 96.61) (end 207.522 95.754) (width 0.25) (layer F.Cu) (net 4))
 (segment (start 212.072 90.66) (end 212.834 91.422) (width 0.25) (layer F.Cu) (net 4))
 (segment (start 212.072 90.424) (end 212.072 90.66) (width 0.25) (layer F.Cu) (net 4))
 (segment (start 212.834 91.422) (end 212.834 91.886) (width 0.25) (layer F.Cu) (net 4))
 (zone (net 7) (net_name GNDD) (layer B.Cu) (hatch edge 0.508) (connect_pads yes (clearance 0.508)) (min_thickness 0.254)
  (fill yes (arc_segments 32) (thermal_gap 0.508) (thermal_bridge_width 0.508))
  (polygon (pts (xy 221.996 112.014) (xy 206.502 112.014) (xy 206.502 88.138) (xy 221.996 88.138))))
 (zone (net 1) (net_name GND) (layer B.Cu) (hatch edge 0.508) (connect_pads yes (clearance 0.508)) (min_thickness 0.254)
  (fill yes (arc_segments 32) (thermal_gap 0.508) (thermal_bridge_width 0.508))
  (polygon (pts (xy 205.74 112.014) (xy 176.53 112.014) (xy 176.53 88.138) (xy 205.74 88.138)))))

